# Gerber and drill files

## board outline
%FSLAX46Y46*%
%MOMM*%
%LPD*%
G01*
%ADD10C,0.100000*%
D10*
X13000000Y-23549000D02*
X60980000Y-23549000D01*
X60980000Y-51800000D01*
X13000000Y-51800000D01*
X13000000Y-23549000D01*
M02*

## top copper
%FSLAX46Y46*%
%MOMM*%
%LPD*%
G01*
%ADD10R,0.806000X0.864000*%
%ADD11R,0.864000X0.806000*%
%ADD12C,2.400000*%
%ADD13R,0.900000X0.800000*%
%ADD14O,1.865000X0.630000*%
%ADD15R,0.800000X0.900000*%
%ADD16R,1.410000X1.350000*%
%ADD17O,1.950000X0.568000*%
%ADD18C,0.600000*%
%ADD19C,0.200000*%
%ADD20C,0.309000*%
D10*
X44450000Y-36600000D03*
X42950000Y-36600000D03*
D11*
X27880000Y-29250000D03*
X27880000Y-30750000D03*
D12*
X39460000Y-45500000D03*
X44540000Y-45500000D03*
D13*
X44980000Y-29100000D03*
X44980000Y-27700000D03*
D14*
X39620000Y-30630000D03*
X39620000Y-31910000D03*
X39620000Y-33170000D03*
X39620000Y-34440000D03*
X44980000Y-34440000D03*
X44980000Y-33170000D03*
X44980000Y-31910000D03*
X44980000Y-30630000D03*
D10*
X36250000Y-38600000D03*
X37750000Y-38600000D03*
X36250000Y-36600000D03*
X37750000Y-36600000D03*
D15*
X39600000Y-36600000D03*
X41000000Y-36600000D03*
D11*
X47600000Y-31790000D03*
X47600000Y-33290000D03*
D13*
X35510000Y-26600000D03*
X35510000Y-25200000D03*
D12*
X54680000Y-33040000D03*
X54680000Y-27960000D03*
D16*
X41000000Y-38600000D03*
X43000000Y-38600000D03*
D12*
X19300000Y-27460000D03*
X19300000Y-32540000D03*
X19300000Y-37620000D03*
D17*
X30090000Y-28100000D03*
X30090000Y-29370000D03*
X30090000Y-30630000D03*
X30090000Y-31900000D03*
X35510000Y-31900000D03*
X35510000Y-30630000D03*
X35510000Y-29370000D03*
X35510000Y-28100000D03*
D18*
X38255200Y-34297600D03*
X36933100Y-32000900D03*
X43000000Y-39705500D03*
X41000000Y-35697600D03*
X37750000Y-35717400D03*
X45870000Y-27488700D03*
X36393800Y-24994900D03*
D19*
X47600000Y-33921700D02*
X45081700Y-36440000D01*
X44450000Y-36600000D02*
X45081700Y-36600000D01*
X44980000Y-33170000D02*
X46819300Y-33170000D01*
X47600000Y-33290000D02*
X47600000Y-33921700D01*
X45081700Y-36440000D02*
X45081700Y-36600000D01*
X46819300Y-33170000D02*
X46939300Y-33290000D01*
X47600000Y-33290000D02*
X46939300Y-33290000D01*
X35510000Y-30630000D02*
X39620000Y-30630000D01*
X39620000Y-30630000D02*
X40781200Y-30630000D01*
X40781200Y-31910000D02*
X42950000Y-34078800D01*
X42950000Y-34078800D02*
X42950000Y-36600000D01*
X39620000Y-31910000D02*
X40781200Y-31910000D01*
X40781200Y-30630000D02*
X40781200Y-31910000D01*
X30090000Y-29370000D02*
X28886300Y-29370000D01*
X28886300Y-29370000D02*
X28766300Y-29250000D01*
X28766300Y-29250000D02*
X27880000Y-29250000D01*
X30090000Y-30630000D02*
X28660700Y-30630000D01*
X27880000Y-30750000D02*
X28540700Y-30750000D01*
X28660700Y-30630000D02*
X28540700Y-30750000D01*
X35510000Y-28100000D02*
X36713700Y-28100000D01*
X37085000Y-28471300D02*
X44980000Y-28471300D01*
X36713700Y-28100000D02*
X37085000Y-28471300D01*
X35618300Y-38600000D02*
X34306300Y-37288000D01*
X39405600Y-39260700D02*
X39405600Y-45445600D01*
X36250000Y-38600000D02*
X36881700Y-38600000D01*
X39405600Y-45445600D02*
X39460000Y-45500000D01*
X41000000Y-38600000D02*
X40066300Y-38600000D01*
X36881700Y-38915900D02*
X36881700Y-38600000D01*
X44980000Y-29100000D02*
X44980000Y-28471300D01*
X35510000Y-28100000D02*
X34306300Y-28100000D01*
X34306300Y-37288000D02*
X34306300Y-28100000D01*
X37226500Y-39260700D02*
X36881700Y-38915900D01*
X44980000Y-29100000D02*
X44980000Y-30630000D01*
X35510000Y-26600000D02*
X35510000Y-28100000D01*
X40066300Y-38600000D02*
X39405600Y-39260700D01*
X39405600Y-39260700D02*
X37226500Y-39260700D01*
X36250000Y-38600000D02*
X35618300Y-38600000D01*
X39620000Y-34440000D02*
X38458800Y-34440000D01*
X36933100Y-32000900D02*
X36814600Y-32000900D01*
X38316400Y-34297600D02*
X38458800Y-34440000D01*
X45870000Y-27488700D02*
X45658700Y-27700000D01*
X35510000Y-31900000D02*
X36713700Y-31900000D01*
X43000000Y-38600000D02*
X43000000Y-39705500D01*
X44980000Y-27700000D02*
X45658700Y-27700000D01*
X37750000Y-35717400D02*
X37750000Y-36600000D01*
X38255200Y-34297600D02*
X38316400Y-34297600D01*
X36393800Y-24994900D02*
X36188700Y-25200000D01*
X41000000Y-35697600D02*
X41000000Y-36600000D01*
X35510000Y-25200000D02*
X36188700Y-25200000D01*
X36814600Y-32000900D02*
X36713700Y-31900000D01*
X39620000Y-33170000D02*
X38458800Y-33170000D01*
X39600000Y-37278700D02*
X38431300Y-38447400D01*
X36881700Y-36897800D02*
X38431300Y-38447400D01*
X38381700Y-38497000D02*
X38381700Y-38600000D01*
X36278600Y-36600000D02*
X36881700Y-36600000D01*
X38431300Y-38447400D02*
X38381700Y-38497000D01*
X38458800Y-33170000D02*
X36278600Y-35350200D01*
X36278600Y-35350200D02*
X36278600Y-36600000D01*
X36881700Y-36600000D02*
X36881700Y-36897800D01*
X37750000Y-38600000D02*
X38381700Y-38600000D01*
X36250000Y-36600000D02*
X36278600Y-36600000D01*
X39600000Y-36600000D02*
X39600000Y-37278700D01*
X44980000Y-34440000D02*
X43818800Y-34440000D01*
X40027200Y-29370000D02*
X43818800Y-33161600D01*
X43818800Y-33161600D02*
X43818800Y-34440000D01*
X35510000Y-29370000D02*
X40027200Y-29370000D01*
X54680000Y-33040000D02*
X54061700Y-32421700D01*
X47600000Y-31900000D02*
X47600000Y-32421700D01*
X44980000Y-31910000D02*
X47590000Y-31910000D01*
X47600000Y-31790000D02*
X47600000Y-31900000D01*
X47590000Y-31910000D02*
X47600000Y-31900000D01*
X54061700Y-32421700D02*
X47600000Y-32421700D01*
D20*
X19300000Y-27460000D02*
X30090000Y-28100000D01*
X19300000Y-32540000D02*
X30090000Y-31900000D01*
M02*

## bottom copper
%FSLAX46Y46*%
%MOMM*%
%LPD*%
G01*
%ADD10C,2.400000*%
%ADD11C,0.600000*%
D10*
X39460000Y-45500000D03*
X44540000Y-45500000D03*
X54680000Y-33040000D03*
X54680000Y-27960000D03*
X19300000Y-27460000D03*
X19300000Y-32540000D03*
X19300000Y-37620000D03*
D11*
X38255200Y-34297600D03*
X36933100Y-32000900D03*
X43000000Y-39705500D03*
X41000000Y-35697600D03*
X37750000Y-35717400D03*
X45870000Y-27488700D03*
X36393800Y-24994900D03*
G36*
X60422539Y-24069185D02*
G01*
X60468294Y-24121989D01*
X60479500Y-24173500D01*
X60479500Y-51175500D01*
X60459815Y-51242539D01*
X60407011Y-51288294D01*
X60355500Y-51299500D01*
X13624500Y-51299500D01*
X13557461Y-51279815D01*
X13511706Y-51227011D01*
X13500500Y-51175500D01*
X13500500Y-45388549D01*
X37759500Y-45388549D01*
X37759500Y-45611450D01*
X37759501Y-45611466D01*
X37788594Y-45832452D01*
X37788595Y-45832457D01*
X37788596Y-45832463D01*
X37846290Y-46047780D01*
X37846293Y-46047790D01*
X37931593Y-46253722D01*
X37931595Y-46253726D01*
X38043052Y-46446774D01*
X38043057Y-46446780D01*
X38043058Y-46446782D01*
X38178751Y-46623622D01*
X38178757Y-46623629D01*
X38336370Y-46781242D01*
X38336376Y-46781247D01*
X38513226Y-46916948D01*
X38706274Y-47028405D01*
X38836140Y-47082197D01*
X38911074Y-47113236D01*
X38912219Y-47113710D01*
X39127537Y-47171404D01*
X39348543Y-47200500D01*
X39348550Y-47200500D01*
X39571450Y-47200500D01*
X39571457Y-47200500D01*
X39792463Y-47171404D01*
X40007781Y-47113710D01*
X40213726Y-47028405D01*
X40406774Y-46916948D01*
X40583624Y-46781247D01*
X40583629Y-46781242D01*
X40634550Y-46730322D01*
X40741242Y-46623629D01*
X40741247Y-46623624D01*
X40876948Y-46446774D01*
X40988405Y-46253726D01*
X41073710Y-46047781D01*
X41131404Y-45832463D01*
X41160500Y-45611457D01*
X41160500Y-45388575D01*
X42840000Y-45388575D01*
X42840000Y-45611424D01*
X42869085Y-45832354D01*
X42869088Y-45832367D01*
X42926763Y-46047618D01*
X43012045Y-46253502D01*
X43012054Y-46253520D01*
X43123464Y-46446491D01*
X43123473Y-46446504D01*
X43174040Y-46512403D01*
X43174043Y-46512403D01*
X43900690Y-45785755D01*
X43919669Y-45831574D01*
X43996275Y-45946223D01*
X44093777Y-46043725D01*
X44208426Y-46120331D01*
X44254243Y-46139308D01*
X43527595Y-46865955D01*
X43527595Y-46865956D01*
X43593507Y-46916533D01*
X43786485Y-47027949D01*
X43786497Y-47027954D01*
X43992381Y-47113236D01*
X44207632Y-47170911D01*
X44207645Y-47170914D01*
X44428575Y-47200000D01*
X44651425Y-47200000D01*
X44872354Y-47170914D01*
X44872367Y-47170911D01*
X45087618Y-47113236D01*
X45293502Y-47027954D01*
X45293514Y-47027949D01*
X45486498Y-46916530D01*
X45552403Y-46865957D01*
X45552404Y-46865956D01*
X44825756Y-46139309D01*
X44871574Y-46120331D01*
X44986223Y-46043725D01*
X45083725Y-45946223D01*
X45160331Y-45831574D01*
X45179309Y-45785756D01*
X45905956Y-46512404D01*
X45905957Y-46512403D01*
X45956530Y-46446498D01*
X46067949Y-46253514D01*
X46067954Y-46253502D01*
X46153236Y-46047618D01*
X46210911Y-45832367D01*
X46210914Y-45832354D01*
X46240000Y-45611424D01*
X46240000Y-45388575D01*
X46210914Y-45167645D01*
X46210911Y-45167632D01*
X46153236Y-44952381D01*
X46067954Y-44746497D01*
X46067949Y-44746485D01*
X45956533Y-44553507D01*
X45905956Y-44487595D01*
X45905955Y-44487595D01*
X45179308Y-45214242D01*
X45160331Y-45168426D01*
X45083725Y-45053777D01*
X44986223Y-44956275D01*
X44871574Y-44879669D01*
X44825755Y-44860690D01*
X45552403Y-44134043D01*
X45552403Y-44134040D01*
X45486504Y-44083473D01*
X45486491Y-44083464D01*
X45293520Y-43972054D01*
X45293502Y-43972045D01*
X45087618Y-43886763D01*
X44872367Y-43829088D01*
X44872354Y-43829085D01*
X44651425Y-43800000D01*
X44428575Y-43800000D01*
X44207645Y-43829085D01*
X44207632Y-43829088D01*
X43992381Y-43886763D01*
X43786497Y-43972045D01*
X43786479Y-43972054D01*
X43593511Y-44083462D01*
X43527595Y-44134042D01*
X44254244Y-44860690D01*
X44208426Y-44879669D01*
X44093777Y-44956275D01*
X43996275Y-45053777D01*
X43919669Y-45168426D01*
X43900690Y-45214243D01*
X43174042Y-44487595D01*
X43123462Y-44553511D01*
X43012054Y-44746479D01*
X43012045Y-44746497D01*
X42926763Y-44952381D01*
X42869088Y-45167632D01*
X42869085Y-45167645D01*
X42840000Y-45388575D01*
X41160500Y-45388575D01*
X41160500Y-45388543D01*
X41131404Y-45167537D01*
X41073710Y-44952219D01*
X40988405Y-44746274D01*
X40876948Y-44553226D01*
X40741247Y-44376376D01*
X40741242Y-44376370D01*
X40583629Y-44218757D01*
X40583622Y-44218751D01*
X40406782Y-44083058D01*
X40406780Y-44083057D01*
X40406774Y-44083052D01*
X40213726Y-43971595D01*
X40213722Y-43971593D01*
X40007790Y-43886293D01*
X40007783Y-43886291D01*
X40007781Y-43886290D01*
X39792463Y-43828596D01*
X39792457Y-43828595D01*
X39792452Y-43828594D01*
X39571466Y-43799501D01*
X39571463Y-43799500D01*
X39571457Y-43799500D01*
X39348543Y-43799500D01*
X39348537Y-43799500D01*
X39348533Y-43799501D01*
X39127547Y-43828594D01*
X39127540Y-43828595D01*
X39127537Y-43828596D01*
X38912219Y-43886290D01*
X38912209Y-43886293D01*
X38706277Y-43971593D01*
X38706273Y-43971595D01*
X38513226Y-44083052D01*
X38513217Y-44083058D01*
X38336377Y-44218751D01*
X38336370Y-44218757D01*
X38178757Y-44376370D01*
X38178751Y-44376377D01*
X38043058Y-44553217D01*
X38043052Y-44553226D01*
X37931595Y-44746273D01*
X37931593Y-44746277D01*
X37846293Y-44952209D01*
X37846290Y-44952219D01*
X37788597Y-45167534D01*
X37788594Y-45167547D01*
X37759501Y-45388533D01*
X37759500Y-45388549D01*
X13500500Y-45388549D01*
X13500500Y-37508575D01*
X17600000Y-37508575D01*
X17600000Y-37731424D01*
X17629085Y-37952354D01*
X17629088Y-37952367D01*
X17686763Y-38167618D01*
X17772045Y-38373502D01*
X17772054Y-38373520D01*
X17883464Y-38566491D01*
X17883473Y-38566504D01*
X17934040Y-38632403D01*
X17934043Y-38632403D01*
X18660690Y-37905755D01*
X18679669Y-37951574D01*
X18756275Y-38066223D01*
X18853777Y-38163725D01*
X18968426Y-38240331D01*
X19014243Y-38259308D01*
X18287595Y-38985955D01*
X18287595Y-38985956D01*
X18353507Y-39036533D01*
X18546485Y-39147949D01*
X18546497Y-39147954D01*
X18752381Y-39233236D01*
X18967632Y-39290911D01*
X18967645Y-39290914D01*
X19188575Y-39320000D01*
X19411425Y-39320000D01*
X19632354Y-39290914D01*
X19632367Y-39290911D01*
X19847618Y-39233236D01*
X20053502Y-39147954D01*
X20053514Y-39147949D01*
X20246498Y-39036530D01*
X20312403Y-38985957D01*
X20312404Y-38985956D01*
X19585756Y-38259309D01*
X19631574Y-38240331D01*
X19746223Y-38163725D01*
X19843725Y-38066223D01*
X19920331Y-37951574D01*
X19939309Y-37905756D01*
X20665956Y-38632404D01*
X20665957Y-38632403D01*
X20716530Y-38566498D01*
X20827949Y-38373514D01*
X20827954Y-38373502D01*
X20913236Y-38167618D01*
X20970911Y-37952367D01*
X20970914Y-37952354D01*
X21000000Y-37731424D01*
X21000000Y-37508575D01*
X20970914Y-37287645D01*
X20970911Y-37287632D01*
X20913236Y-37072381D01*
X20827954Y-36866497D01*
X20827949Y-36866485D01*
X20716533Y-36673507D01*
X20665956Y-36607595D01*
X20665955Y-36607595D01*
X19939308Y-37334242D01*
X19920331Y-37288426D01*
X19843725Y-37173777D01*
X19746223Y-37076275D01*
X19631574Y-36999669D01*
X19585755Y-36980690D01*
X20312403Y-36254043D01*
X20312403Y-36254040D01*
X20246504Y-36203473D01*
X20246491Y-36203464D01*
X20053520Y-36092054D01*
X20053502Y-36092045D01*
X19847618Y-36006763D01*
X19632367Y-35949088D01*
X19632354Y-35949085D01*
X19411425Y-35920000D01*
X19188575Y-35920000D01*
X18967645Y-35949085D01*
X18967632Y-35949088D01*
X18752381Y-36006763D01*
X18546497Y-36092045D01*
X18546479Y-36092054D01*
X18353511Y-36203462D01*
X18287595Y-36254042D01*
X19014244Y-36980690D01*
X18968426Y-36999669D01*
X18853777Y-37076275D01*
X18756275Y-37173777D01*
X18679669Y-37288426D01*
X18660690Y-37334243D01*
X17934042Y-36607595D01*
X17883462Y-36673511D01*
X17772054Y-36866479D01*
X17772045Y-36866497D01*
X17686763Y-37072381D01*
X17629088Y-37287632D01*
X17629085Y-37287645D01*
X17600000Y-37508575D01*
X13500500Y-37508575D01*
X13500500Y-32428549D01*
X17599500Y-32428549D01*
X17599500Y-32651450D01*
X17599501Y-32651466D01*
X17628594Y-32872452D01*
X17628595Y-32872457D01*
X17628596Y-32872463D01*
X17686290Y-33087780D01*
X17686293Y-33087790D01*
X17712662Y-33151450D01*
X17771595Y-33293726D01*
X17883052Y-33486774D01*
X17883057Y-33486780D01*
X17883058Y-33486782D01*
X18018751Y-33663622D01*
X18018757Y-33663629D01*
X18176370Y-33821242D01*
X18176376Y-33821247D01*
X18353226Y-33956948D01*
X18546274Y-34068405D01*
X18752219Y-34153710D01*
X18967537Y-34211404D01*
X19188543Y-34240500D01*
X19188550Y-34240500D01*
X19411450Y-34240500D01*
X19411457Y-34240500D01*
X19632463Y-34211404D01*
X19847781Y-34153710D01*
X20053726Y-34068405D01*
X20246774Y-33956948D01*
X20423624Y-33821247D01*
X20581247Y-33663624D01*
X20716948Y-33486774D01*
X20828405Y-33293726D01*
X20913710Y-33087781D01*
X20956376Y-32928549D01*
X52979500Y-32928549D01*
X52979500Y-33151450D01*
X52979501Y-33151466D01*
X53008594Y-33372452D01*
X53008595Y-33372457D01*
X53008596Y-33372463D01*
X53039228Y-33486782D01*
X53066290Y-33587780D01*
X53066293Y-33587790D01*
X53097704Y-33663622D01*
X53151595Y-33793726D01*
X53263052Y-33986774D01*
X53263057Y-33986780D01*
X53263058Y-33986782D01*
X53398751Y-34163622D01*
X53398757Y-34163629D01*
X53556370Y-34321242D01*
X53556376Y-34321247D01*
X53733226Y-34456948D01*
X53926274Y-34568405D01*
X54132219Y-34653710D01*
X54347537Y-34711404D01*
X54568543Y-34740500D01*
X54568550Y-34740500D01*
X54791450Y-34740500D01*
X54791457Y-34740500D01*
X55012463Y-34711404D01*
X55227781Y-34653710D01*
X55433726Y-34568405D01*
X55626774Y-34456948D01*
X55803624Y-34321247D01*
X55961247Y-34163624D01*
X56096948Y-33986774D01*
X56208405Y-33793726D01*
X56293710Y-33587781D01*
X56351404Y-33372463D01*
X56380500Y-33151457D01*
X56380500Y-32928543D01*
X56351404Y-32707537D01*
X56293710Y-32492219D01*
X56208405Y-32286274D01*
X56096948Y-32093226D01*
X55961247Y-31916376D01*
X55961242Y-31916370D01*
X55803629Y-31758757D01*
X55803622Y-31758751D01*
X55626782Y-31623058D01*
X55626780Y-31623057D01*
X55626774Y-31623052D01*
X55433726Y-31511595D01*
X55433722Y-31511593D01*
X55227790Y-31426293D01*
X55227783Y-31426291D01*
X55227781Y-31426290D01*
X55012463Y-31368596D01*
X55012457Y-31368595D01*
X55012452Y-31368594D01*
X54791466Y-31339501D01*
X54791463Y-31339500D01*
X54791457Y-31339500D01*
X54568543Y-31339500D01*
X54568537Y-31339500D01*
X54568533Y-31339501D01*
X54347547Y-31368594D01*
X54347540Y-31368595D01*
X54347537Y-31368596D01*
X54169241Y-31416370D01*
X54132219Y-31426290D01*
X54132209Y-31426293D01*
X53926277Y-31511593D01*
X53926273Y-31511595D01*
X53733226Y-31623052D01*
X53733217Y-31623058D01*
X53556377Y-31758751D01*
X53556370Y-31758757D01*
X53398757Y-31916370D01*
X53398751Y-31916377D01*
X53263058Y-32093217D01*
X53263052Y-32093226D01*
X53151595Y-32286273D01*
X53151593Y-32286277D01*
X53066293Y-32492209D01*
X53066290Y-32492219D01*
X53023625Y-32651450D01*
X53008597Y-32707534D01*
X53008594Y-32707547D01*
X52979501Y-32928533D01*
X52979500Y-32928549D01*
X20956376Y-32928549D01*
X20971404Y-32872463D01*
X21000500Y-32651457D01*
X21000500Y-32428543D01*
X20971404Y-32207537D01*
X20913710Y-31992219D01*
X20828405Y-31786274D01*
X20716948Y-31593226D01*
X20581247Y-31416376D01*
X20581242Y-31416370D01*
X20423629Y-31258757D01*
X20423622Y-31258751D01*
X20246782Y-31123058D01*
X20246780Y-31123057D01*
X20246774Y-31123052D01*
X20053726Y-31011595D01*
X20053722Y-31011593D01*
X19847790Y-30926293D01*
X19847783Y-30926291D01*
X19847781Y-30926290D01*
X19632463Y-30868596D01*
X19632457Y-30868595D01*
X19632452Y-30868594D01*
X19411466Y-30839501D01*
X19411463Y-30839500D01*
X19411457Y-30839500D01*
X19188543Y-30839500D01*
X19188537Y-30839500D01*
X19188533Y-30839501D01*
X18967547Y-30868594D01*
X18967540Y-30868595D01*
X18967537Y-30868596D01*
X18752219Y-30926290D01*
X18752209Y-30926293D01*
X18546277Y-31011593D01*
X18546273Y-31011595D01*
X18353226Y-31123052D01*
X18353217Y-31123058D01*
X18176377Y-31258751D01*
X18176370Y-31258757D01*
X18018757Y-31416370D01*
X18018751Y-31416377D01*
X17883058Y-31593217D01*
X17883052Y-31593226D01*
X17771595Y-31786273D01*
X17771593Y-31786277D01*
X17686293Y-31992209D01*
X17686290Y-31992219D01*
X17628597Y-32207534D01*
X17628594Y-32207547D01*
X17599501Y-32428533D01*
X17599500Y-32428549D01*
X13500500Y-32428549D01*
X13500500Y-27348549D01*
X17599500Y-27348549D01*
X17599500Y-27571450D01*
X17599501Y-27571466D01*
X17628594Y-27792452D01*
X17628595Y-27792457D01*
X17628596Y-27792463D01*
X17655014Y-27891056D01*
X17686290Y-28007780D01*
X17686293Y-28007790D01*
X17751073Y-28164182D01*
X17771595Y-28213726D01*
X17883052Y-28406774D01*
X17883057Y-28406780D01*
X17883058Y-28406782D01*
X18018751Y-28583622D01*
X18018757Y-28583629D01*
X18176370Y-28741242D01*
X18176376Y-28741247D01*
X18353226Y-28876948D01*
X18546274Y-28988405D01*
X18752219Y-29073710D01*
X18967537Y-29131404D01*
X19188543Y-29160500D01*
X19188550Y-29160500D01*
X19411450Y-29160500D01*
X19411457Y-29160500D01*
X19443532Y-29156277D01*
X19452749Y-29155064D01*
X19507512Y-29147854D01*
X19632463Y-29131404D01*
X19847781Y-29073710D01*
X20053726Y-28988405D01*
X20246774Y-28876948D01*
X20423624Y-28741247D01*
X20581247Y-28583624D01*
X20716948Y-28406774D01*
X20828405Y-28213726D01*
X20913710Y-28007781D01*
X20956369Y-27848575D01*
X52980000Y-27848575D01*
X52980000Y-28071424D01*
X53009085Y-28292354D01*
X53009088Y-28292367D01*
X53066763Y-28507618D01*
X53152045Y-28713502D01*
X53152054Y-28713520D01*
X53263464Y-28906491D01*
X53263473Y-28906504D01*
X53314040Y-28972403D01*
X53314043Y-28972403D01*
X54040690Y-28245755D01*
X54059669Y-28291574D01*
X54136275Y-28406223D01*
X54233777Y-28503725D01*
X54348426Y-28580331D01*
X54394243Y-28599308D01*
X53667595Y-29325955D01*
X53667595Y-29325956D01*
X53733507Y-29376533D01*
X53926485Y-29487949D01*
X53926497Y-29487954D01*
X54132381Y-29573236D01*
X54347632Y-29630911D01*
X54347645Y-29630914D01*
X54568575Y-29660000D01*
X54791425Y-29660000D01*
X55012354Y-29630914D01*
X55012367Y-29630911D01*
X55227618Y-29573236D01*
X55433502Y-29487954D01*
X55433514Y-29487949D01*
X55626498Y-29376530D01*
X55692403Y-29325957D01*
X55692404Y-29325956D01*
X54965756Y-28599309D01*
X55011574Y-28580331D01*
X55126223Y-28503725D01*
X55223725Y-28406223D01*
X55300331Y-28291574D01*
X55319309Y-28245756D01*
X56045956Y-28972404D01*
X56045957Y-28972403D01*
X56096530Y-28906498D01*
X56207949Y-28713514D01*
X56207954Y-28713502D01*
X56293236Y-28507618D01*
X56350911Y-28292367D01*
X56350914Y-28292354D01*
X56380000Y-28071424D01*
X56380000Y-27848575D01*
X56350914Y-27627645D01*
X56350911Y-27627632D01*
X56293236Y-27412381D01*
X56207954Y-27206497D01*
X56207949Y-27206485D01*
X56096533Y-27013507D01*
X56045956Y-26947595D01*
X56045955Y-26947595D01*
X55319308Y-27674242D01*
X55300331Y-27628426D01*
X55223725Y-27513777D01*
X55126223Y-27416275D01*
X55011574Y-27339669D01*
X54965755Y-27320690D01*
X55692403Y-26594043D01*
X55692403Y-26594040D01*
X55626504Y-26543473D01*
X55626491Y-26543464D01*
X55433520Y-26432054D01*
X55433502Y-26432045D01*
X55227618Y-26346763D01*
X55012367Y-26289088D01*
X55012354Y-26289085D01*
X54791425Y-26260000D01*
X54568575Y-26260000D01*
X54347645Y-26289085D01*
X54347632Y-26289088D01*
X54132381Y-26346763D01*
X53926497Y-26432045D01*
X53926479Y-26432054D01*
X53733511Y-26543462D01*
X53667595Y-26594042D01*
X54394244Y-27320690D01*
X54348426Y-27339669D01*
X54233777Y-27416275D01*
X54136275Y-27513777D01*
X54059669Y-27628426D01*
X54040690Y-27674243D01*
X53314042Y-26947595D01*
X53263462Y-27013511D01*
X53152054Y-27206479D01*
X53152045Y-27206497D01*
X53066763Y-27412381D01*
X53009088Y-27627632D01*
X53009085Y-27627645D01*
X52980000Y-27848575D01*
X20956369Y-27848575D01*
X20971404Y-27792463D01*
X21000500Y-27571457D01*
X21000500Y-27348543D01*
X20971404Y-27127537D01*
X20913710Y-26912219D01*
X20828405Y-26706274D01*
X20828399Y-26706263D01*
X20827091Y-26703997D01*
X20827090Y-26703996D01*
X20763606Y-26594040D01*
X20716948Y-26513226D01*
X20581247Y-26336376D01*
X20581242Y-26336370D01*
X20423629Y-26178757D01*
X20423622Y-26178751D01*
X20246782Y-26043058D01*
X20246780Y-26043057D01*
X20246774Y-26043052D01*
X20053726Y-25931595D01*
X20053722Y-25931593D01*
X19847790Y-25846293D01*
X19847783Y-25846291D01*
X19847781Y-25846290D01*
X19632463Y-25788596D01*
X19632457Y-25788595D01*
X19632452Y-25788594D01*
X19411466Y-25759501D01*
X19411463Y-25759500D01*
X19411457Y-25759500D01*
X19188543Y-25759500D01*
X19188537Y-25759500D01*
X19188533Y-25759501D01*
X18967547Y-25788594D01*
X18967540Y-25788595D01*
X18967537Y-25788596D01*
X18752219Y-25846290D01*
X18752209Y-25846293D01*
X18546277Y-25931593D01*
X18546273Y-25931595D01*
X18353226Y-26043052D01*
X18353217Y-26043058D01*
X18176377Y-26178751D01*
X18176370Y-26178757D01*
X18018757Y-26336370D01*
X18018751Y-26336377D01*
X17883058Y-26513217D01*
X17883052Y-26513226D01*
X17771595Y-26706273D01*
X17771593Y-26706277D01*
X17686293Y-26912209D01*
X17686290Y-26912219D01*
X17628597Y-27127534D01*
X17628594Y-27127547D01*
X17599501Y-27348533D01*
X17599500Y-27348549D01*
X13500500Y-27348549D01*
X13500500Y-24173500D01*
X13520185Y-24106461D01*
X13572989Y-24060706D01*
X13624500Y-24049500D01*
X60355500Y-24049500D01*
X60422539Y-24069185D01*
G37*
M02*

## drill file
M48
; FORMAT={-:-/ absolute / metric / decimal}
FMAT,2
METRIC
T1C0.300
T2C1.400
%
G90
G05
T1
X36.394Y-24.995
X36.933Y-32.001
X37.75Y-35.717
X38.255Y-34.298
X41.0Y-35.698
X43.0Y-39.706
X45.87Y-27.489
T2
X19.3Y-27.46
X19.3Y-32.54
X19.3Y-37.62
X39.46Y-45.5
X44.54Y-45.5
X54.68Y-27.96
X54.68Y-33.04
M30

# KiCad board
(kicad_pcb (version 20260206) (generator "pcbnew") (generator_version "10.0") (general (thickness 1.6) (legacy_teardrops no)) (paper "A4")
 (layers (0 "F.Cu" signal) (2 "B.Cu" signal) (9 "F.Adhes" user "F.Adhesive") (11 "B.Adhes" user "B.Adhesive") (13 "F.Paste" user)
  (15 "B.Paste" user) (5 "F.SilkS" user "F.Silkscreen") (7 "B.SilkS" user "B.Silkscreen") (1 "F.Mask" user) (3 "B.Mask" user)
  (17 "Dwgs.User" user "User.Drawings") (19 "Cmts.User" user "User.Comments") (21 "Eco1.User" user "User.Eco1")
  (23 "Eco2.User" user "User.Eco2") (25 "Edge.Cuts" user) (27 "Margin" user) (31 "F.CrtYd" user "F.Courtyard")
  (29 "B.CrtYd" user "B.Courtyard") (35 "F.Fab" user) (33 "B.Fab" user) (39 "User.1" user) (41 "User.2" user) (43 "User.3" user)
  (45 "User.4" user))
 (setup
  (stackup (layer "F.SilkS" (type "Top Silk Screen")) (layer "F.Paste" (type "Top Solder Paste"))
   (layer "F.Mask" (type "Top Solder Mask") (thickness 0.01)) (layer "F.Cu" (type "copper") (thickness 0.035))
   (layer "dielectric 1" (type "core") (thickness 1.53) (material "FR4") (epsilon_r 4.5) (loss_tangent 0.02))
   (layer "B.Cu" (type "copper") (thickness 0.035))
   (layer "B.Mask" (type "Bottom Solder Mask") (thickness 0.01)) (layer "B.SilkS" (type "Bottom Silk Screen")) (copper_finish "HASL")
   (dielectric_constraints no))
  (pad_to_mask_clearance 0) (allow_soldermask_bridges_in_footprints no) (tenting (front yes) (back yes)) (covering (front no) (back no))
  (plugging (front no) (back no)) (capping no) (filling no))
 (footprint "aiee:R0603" (layer "F.Cu") (at 43.7 36.6 180)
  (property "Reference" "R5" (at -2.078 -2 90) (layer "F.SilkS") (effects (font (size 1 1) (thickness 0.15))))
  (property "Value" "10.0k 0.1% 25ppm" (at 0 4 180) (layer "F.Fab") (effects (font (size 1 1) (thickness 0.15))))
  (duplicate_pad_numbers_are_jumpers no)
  (pad "1" smd rect (at -0.75 0 180) (size 0.806 0.864) (layers "F.Cu" "F.Mask" "F.Paste") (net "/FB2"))
  (pad "2" smd rect (at 0.75 0 180) (size 0.806 0.864) (layers "F.Cu" "F.Mask" "F.Paste") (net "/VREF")))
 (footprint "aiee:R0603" (layer "F.Cu") (at 27.88 30 -90)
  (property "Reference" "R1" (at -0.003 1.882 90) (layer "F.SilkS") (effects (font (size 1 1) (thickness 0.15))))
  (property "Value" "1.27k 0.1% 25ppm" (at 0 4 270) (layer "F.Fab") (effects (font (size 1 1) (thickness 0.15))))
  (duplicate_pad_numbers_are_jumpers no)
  (pad "1" smd rect (at -0.75 0 270) (size 0.806 0.864) (layers "F.Cu" "F.Mask" "F.Paste") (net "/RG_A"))
  (pad "2" smd rect (at 0.75 0 270) (size 0.806 0.864) (layers "F.Cu" "F.Mask" "F.Paste") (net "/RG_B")))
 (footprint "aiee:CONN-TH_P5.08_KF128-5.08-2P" (layer "F.Cu") (at 42 45.5)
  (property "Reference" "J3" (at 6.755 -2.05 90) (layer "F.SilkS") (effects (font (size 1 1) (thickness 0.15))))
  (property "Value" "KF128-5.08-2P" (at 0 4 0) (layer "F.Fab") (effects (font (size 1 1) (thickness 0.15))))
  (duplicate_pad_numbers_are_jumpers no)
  (pad "1" thru_hole circle (at -2.54 0) (size 2.4 2.4) (drill 1.399998) (layers "*.Cu" "*.Mask") (remove_unused_layers no) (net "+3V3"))
  (pad "2" thru_hole circle (at 2.54 0) (size 2.4 2.4) (drill 1.399998) (layers "*.Cu" "*.Mask") (remove_unused_layers no) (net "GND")))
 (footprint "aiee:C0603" (layer "F.Cu") (at 44.98 28.4 90)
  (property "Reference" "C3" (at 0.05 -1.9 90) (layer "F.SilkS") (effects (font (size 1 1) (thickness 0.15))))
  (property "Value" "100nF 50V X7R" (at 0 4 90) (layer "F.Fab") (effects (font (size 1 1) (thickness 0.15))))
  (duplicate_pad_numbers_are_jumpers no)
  (pad "1" smd rect (at -0.7 0 90) (size 0.8 0.9) (layers "F.Cu" "F.Mask" "F.Paste") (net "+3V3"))
  (pad "2" smd rect (at 0.7 0 90) (size 0.8 0.9) (layers "F.Cu" "F.Mask" "F.Paste") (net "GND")))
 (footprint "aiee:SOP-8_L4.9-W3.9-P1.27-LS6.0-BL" (layer "F.Cu") (at 42.3 32.54 -90)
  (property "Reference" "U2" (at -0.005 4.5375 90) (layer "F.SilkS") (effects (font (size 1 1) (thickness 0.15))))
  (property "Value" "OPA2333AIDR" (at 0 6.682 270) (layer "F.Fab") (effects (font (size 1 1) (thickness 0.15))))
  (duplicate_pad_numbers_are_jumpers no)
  (pad "1" smd oval (at -1.91 2.68 270) (size 0.63 1.865) (layers "F.Cu" "F.Mask" "F.Paste") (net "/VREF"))
  (pad "2" smd oval (at -0.63 2.68 270) (size 0.63 1.865) (layers "F.Cu" "F.Mask" "F.Paste") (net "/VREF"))
  (pad "3" smd oval (at 0.63 2.68 270) (size 0.63 1.865) (layers "F.Cu" "F.Mask" "F.Paste") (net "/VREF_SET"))
  (pad "4" smd oval (at 1.9 2.68 270) (size 0.63 1.865) (layers "F.Cu" "F.Mask" "F.Paste") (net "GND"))
  (pad "5" smd oval (at 1.9 -2.68 270) (size 0.63 1.865) (layers "F.Cu" "F.Mask" "F.Paste") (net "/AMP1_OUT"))
  (pad "6" smd oval (at 0.63 -2.68 270) (size 0.63 1.865) (layers "F.Cu" "F.Mask" "F.Paste") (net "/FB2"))
  (pad "7" smd oval (at -0.63 -2.68 270) (size 0.63 1.865) (layers "F.Cu" "F.Mask" "F.Paste") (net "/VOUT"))
  (pad "8" smd oval (at -1.91 -2.68 270) (size 0.63 1.865) (layers "F.Cu" "F.Mask" "F.Paste") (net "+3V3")))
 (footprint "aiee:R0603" (layer "F.Cu") (at 37 38.6)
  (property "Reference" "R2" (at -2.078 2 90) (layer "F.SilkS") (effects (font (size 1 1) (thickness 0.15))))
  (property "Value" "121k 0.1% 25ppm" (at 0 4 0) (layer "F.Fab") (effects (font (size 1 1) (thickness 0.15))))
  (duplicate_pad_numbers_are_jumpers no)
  (pad "1" smd rect (at -0.75 0) (size 0.806 0.864) (layers "F.Cu" "F.Mask" "F.Paste") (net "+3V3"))
  (pad "2" smd rect (at 0.75 0) (size 0.806 0.864) (layers "F.Cu" "F.Mask" "F.Paste") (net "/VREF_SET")))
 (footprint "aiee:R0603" (layer "F.Cu") (at 37 36.6)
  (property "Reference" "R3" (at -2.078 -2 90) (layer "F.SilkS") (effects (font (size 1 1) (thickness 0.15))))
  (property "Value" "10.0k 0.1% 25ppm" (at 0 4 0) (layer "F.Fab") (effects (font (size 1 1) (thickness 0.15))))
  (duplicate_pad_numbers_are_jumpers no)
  (pad "1" smd rect (at -0.75 0) (size 0.806 0.864) (layers "F.Cu" "F.Mask" "F.Paste") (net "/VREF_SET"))
  (pad "2" smd rect (at 0.75 0) (size 0.806 0.864) (layers "F.Cu" "F.Mask" "F.Paste") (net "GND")))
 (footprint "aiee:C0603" (layer "F.Cu") (at 40.3 36.6)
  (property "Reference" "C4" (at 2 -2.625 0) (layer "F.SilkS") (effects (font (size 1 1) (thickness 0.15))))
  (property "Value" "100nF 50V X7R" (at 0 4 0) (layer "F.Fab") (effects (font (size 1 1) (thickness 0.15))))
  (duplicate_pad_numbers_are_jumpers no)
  (pad "1" smd rect (at -0.7 0) (size 0.8 0.9) (layers "F.Cu" "F.Mask" "F.Paste") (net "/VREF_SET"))
  (pad "2" smd rect (at 0.7 0) (size 0.8 0.9) (layers "F.Cu" "F.Mask" "F.Paste") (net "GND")))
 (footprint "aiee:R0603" (layer "F.Cu") (at 47.6 32.54 -90)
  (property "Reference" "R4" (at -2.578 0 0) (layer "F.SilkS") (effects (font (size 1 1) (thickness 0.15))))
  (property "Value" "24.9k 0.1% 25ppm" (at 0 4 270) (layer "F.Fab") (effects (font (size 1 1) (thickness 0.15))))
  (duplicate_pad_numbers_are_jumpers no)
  (pad "1" smd rect (at -0.75 0 270) (size 0.806 0.864) (layers "F.Cu" "F.Mask" "F.Paste") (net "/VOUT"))
  (pad "2" smd rect (at 0.75 0 270) (size 0.806 0.864) (layers "F.Cu" "F.Mask" "F.Paste") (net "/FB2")))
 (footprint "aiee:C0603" (layer "F.Cu") (at 35.51 25.9 90)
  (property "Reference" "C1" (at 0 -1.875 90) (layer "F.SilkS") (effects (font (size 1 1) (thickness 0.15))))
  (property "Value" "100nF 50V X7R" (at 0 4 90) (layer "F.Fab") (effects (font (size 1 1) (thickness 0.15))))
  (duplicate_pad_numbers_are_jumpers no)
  (pad "1" smd rect (at -0.7 0 90) (size 0.8 0.9) (layers "F.Cu" "F.Mask" "F.Paste") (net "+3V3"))
  (pad "2" smd rect (at 0.7 0 90) (size 0.8 0.9) (layers "F.Cu" "F.Mask" "F.Paste") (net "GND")))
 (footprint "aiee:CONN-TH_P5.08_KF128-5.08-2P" (layer "F.Cu") (at 54.68 30.5 90)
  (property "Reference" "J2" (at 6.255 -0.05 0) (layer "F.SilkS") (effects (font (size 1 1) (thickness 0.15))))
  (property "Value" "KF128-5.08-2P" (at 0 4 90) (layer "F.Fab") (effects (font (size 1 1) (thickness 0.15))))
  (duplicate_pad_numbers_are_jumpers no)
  (pad "1" thru_hole circle (at -2.54 0 90) (size 2.4 2.4) (drill 1.399998) (layers "*.Cu" "*.Mask") (remove_unused_layers no) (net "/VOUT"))
  (pad "2" thru_hole circle (at 2.54 0 90) (size 2.4 2.4) (drill 1.399998) (layers "*.Cu" "*.Mask") (remove_unused_layers no) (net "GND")))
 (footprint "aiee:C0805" (layer "F.Cu") (at 42 38.6)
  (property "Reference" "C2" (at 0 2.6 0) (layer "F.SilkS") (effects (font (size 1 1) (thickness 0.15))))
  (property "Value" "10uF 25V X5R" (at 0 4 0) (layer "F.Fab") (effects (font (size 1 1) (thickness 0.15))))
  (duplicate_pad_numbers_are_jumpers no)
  (pad "1" smd rect (at -1 0) (size 1.41 1.35) (layers "F.Cu" "F.Mask" "F.Paste") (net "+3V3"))
  (pad "2" smd rect (at 1 0) (size 1.41 1.35) (layers "F.Cu" "F.Mask" "F.Paste") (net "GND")))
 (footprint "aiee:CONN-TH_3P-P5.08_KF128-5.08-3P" (layer "F.Cu") (at 19.3 32.54 -90)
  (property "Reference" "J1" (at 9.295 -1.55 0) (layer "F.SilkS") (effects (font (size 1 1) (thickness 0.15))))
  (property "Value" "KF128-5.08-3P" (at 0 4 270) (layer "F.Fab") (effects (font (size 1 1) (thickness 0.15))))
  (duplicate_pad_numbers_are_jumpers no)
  (pad "1" thru_hole circle (at -5.08 0 270) (size 2.4 2.4) (drill 1.399998) (layers "*.Cu" "*.Mask") (remove_unused_layers no)
   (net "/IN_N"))
  (pad "2" thru_hole circle (at 0 0 270) (size 2.4 2.4) (drill 1.399998) (layers "*.Cu" "*.Mask") (remove_unused_layers no) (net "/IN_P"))
  (pad "3" thru_hole circle (at 5.08 0 270) (size 2.4 2.4) (drill 1.399998) (layers "*.Cu" "*.Mask") (remove_unused_layers no) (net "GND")))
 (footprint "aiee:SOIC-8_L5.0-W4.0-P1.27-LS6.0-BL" (layer "F.Cu") (at 32.8 30 -90)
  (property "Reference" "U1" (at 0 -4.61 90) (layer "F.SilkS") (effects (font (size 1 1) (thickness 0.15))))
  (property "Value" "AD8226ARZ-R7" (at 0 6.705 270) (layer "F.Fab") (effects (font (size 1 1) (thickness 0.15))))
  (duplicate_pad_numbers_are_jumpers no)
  (pad "1" smd oval (at -1.9 2.71 270) (size 0.568 1.95) (layers "F.Cu" "F.Mask" "F.Paste") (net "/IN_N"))
  (pad "2" smd oval (at -0.63 2.71 270) (size 0.568 1.95) (layers "F.Cu" "F.Mask" "F.Paste") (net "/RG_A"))
  (pad "3" smd oval (at 0.63 2.71 270) (size 0.568 1.95) (layers "F.Cu" "F.Mask" "F.Paste") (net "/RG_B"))
  (pad "4" smd oval (at 1.9 2.71 270) (size 0.568 1.95) (layers "F.Cu" "F.Mask" "F.Paste") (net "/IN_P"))
  (pad "5" smd oval (at 1.9 -2.71 270) (size 0.568 1.95) (layers "F.Cu" "F.Mask" "F.Paste") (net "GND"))
  (pad "6" smd oval (at 0.63 -2.71 270) (size 0.568 1.95) (layers "F.Cu" "F.Mask" "F.Paste") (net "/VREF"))
  (pad "7" smd oval (at -0.63 -2.71 270) (size 0.568 1.95) (layers "F.Cu" "F.Mask" "F.Paste") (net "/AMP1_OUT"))
  (pad "8" smd oval (at -1.9 -2.71 270) (size 0.568 1.95) (layers "F.Cu" "F.Mask" "F.Paste") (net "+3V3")))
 (gr_rect (start 13 23.549) (end 60.98 51.8) (stroke (width 0.1) (type default)) (fill no) (layer "Edge.Cuts"))
 (segment (start 47.6 33.9217) (end 45.0817 36.44) (width 0.2) (layer "F.Cu") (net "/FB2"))
 (segment (start 44.45 36.6) (end 45.0817 36.6) (width 0.2) (layer "F.Cu") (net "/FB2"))
 (segment (start 44.98 33.17) (end 46.8193 33.17) (width 0.2) (layer "F.Cu") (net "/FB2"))
 (segment (start 47.6 33.29) (end 47.6 33.9217) (width 0.2) (layer "F.Cu") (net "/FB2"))
 (segment (start 45.0817 36.44) (end 45.0817 36.6) (width 0.2) (layer "F.Cu") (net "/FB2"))
 (segment (start 46.8193 33.17) (end 46.9393 33.29) (width 0.2) (layer "F.Cu") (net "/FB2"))
 (segment (start 47.6 33.29) (end 46.9393 33.29) (width 0.2) (layer "F.Cu") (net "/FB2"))
 (segment (start 35.51 30.63) (end 39.62 30.63) (width 0.2) (layer "F.Cu") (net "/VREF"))
 (segment (start 39.62 30.63) (end 40.7812 30.63) (width 0.2) (layer "F.Cu") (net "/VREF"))
 (segment (start 40.7812 31.91) (end 42.95 34.0788) (width 0.2) (layer "F.Cu") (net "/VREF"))
 (segment (start 42.95 34.0788) (end 42.95 36.6) (width 0.2) (layer "F.Cu") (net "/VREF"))
 (segment (start 39.62 31.91) (end 40.7812 31.91) (width 0.2) (layer "F.Cu") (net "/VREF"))
 (segment (start 40.7812 30.63) (end 40.7812 31.91) (width 0.2) (layer "F.Cu") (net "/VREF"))
 (segment (start 30.09 29.37) (end 28.8863 29.37) (width 0.2) (layer "F.Cu") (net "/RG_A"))
 (segment (start 28.8863 29.37) (end 28.7663 29.25) (width 0.2) (layer "F.Cu") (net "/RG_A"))
 (segment (start 28.7663 29.25) (end 27.88 29.25) (width 0.2) (layer "F.Cu") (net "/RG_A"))
 (segment (start 30.09 30.63) (end 28.6607 30.63) (width 0.2) (layer "F.Cu") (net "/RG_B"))
 (segment (start 27.88 30.75) (end 28.5407 30.75) (width 0.2) (layer "F.Cu") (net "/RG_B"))
 (segment (start 28.6607 30.63) (end 28.5407 30.75) (width 0.2) (layer "F.Cu") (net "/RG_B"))
 (segment (start 35.51 28.1) (end 36.7137 28.1) (width 0.2) (layer "F.Cu") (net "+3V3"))
 (segment (start 37.085 28.4713) (end 44.98 28.4713) (width 0.2) (layer "F.Cu") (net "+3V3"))
 (segment (start 36.7137 28.1) (end 37.085 28.4713) (width 0.2) (layer "F.Cu") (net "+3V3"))
 (segment (start 35.6183 38.6) (end 34.3063 37.288) (width 0.2) (layer "F.Cu") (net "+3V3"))
 (segment (start 39.4056 39.2607) (end 39.4056 45.4456) (width 0.2) (layer "F.Cu") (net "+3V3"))
 (segment (start 36.25 38.6) (end 36.8817 38.6) (width 0.2) (layer "F.Cu") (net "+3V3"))
 (segment (start 39.4056 45.4456) (end 39.46 45.5) (width 0.2) (layer "F.Cu") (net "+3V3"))
 (segment (start 41 38.6) (end 40.0663 38.6) (width 0.2) (layer "F.Cu") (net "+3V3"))
 (segment (start 36.8817 38.9159) (end 36.8817 38.6) (width 0.2) (layer "F.Cu") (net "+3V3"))
 (segment (start 44.98 29.1) (end 44.98 28.4713) (width 0.2) (layer "F.Cu") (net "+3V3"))
 (segment (start 35.51 28.1) (end 34.3063 28.1) (width 0.2) (layer "F.Cu") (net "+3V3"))
 (segment (start 34.3063 37.288) (end 34.3063 28.1) (width 0.2) (layer "F.Cu") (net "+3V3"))
 (segment (start 37.2265 39.2607) (end 36.8817 38.9159) (width 0.2) (layer "F.Cu") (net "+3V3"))
 (segment (start 44.98 29.1) (end 44.98 30.63) (width 0.2) (layer "F.Cu") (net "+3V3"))
 (segment (start 35.51 26.6) (end 35.51 28.1) (width 0.2) (layer "F.Cu") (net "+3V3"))
 (segment (start 40.0663 38.6) (end 39.4056 39.2607) (width 0.2) (layer "F.Cu") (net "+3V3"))
 (segment (start 39.4056 39.2607) (end 37.2265 39.2607) (width 0.2) (layer "F.Cu") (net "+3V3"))
 (segment (start 36.25 38.6) (end 35.6183 38.6) (width 0.2) (layer "F.Cu") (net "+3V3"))
 (segment (start 39.62 34.44) (end 38.4588 34.44) (width 0.2) (layer "F.Cu") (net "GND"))
 (segment (start 36.9331 32.0009) (end 36.8146 32.0009) (width 0.2) (layer "F.Cu") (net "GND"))
 (segment (start 38.3164 34.2976) (end 38.4588 34.44) (width 0.2) (layer "F.Cu") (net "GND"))
 (segment (start 45.87 27.4887) (end 45.6587 27.7) (width 0.2) (layer "F.Cu") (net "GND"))
 (segment (start 35.51 31.9) (end 36.7137 31.9) (width 0.2) (layer "F.Cu") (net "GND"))
 (segment (start 43 38.6) (end 43 39.7055) (width 0.2) (layer "F.Cu") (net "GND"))
 (segment (start 44.98 27.7) (end 45.6587 27.7) (width 0.2) (layer "F.Cu") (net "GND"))
 (segment (start 37.75 35.7174) (end 37.75 36.6) (width 0.2) (layer "F.Cu") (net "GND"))
 (segment (start 38.2552 34.2976) (end 38.3164 34.2976) (width 0.2) (layer "F.Cu") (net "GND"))
 (segment (start 36.3938 24.9949) (end 36.1887 25.2) (width 0.2) (layer "F.Cu") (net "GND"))
 (segment (start 41 35.6976) (end 41 36.6) (width 0.2) (layer "F.Cu") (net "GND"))
 (segment (start 35.51 25.2) (end 36.1887 25.2) (width 0.2) (layer "F.Cu") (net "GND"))
 (segment (start 36.8146 32.0009) (end 36.7137 31.9) (width 0.2) (layer "F.Cu") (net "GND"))
 (via (at 38.2552 34.2976) (size 0.6) (drill 0.3) (layers "F.Cu" "B.Cu") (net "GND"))
 (via (at 36.9331 32.0009) (size 0.6) (drill 0.3) (layers "F.Cu" "B.Cu") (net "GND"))
 (via (at 43 39.7055) (size 0.6) (drill 0.3) (layers "F.Cu" "B.Cu") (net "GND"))
 (via (at 41 35.6976) (size 0.6) (drill 0.3) (layers "F.Cu" "B.Cu") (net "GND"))
 (via (at 37.75 35.7174) (size 0.6) (drill 0.3) (layers "F.Cu" "B.Cu") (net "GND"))
 (via (at 45.87 27.4887) (size 0.6) (drill 0.3) (layers "F.Cu" "B.Cu") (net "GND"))
 (via (at 36.3938 24.9949) (size 0.6) (drill 0.3) (layers "F.Cu" "B.Cu") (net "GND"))
 (segment (start 39.62 33.17) (end 38.4588 33.17) (width 0.2) (layer "F.Cu") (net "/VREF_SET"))
 (segment (start 39.6 37.2787) (end 38.4313 38.4474) (width 0.2) (layer "F.Cu") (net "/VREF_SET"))
 (segment (start 36.8817 36.8978) (end 38.4313 38.4474) (width 0.2) (layer "F.Cu") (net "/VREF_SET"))
 (segment (start 38.3817 38.497) (end 38.3817 38.6) (width 0.2) (layer "F.Cu") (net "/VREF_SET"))
 (segment (start 36.2786 36.6) (end 36.8817 36.6) (width 0.2) (layer "F.Cu") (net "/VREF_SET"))
 (segment (start 38.4313 38.4474) (end 38.3817 38.497) (width 0.2) (layer "F.Cu") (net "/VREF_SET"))
 (segment (start 38.4588 33.17) (end 36.2786 35.3502) (width 0.2) (layer "F.Cu") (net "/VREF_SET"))
 (segment (start 36.2786 35.3502) (end 36.2786 36.6) (width 0.2) (layer "F.Cu") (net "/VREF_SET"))
 (segment (start 36.8817 36.6) (end 36.8817 36.8978) (width 0.2) (layer "F.Cu") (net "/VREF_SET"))
 (segment (start 37.75 38.6) (end 38.3817 38.6) (width 0.2) (layer "F.Cu") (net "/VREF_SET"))
 (segment (start 36.25 36.6) (end 36.2786 36.6) (width 0.2) (layer "F.Cu") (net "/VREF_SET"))
 (segment (start 39.6 36.6) (end 39.6 37.2787) (width 0.2) (layer "F.Cu") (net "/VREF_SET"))
 (segment (start 44.98 34.44) (end 43.8188 34.44) (width 0.2) (layer "F.Cu") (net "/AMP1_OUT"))
 (segment (start 40.0272 29.37) (end 43.8188 33.1616) (width 0.2) (layer "F.Cu") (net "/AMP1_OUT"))
 (segment (start 43.8188 33.1616) (end 43.8188 34.44) (width 0.2) (layer "F.Cu") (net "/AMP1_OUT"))
 (segment (start 35.51 29.37) (end 40.0272 29.37) (width 0.2) (layer "F.Cu") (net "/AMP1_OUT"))
 (segment (start 54.68 33.04) (end 54.0617 32.4217) (width 0.2) (layer "F.Cu") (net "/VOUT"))
 (segment (start 47.6 31.9) (end 47.6 32.4217) (width 0.2) (layer "F.Cu") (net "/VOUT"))
 (segment (start 44.98 31.91) (end 47.59 31.91) (width 0.2) (layer "F.Cu") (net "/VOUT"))
 (segment (start 47.6 31.79) (end 47.6 31.9) (width 0.2) (layer "F.Cu") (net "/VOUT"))
 (segment (start 47.59 31.91) (end 47.6 31.9) (width 0.2) (layer "F.Cu") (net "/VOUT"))
 (segment (start 54.0617 32.4217) (end 47.6 32.4217) (width 0.2) (layer "F.Cu") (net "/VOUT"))
 (segment (start 19.3 27.46) (end 30.09 28.1) (width 0.309) (layer "F.Cu") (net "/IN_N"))
 (segment (start 19.3 32.54) (end 30.09 31.9) (width 0.309) (layer "F.Cu") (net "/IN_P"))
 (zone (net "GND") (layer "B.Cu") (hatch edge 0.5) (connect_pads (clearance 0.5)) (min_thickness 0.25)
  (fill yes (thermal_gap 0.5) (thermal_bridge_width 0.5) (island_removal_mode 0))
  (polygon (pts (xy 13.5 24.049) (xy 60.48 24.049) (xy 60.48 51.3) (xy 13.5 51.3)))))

